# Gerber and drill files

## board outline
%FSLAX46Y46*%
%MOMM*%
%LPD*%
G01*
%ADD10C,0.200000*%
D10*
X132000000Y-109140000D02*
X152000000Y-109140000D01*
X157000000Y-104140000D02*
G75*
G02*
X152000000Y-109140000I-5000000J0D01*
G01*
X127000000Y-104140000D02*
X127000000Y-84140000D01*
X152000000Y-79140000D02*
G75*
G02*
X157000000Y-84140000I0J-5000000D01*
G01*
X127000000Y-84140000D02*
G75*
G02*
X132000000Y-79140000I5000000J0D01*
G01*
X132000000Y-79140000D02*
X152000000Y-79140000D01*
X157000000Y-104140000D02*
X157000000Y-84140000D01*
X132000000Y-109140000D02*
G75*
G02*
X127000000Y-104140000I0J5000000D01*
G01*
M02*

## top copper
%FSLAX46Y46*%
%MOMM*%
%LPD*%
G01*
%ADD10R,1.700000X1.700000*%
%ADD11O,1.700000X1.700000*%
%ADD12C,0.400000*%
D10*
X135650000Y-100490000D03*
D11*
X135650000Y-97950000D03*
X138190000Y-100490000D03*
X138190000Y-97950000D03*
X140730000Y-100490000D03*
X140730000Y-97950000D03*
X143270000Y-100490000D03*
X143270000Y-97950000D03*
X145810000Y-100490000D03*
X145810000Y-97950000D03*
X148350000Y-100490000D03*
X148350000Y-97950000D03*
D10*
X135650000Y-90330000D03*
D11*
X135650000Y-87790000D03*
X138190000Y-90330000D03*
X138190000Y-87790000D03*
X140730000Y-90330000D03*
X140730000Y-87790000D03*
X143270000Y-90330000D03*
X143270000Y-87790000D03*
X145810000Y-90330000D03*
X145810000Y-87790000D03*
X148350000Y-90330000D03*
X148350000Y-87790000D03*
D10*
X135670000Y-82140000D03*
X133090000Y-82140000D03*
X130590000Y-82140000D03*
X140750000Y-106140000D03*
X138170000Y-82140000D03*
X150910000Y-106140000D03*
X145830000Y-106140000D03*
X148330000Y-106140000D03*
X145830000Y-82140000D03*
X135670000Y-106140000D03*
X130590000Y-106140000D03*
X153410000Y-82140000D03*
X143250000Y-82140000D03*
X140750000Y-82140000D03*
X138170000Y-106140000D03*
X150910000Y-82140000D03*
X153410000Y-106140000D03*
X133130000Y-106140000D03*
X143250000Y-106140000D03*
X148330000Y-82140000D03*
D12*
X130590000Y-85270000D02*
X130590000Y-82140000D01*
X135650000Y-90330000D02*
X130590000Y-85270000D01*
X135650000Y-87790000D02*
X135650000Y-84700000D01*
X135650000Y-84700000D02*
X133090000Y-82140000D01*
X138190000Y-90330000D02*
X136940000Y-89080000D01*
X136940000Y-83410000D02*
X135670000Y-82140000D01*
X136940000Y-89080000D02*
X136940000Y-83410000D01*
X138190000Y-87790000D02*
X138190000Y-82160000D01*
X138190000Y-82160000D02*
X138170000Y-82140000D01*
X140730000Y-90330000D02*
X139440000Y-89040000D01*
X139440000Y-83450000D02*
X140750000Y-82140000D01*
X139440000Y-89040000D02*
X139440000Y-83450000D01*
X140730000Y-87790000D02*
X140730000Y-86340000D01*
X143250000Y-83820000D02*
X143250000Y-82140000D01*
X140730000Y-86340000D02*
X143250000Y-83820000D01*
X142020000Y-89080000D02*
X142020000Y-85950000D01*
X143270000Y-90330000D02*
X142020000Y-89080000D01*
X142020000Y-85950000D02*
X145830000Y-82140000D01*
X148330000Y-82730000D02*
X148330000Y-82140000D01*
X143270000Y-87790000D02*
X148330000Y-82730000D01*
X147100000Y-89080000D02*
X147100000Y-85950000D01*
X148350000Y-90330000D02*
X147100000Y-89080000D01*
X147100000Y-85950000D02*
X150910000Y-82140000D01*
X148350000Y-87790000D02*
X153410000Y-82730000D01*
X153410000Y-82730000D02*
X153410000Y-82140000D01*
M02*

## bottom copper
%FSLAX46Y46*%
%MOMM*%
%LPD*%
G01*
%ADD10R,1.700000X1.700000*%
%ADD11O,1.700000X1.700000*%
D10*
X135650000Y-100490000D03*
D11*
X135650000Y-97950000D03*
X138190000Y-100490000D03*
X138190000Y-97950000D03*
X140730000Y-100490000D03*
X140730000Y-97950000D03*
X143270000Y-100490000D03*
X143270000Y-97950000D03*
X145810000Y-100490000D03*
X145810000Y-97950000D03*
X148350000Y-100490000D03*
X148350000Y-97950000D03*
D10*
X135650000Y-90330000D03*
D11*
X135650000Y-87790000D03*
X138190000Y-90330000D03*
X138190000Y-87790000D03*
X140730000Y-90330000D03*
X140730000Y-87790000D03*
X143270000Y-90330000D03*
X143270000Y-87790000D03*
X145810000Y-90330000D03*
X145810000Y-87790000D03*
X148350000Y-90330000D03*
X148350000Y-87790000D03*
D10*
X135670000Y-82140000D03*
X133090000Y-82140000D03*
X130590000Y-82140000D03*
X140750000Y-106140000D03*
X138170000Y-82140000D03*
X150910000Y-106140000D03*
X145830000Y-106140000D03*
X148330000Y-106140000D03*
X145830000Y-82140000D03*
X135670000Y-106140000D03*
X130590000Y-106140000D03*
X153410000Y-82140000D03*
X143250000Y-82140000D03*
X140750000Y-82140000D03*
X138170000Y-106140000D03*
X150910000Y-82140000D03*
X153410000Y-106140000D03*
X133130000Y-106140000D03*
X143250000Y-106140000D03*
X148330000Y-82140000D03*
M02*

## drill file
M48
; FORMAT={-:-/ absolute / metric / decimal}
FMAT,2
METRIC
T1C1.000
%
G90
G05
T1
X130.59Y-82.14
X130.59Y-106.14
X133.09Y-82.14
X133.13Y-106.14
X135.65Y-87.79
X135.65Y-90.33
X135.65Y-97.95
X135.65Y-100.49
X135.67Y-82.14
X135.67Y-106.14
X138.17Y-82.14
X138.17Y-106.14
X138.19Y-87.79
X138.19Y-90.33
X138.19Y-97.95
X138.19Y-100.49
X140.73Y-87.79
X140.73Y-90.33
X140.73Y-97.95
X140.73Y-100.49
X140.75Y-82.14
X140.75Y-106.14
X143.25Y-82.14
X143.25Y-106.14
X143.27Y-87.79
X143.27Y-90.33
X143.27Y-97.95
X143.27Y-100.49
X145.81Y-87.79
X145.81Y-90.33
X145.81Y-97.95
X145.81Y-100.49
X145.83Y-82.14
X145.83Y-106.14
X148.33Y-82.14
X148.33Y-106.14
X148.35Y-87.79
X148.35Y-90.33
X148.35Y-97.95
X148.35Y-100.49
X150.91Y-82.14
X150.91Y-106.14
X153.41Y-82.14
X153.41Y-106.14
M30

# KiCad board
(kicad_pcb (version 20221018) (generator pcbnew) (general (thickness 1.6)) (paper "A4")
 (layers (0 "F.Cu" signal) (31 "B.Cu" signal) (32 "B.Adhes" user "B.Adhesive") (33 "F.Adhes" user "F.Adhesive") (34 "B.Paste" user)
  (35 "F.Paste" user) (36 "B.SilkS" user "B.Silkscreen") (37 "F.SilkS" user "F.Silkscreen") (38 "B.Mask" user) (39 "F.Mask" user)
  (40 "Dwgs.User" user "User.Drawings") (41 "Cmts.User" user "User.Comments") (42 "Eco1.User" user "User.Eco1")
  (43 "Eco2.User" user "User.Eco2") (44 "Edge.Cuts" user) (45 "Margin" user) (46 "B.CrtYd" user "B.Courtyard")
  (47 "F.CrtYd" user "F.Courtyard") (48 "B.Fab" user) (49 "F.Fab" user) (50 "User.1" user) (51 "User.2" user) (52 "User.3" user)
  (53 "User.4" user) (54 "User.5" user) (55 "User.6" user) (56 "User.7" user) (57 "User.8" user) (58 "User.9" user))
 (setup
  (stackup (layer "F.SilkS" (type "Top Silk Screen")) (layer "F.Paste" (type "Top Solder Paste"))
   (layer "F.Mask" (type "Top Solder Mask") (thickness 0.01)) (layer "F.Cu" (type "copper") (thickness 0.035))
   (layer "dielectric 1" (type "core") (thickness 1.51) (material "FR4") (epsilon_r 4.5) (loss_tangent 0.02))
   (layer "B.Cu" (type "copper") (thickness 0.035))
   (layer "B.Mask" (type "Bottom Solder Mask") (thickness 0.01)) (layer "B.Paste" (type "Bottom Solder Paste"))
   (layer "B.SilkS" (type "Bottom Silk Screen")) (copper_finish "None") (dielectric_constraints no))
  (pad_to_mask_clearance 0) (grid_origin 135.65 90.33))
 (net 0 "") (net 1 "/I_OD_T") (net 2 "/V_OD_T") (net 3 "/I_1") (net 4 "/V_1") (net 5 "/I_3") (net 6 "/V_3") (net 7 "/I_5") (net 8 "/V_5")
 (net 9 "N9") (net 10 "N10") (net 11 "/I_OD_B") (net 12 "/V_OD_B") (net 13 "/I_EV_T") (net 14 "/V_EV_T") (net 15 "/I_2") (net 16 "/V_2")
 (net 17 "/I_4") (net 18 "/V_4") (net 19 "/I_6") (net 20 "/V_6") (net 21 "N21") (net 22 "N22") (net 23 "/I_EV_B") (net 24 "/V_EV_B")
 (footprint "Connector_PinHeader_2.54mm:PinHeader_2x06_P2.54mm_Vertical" (layer "F.Cu") (at 135.65 100.49 90)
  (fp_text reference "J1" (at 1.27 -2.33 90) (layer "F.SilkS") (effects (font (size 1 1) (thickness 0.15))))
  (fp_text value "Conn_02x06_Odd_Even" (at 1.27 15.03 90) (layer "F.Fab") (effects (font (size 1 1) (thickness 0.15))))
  (pad "1" thru_hole rect (at 0 0 90) (size 1.7 1.7) (drill 1) (layers "*.Cu" "*.Mask") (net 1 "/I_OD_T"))
  (pad "2" thru_hole oval (at 2.54 0 90) (size 1.7 1.7) (drill 1) (layers "*.Cu" "*.Mask") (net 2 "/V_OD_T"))
  (pad "3" thru_hole oval (at 0 2.54 90) (size 1.7 1.7) (drill 1) (layers "*.Cu" "*.Mask") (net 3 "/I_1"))
  (pad "4" thru_hole oval (at 2.54 2.54 90) (size 1.7 1.7) (drill 1) (layers "*.Cu" "*.Mask") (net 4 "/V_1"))
  (pad "5" thru_hole oval (at 0 5.08 90) (size 1.7 1.7) (drill 1) (layers "*.Cu" "*.Mask") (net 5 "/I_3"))
  (pad "6" thru_hole oval (at 2.54 5.08 90) (size 1.7 1.7) (drill 1) (layers "*.Cu" "*.Mask") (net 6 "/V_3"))
  (pad "7" thru_hole oval (at 0 7.62 90) (size 1.7 1.7) (drill 1) (layers "*.Cu" "*.Mask") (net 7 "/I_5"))
  (pad "8" thru_hole oval (at 2.54 7.62 90) (size 1.7 1.7) (drill 1) (layers "*.Cu" "*.Mask") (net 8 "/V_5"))
  (pad "9" thru_hole oval (at 0 10.16 90) (size 1.7 1.7) (drill 1) (layers "*.Cu" "*.Mask") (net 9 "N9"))
  (pad "10" thru_hole oval (at 2.54 10.16 90) (size 1.7 1.7) (drill 1) (layers "*.Cu" "*.Mask") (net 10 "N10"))
  (pad "11" thru_hole oval (at 0 12.7 90) (size 1.7 1.7) (drill 1) (layers "*.Cu" "*.Mask") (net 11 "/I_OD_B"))
  (pad "12" thru_hole oval (at 2.54 12.7 90) (size 1.7 1.7) (drill 1) (layers "*.Cu" "*.Mask") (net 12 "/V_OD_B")))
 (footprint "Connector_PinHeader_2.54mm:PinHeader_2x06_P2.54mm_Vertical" (layer "F.Cu") (at 135.65 90.33 90)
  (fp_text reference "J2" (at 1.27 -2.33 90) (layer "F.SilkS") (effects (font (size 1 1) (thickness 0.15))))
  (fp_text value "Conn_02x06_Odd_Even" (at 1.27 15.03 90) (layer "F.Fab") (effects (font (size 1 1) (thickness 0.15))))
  (pad "1" thru_hole rect (at 0 0 90) (size 1.7 1.7) (drill 1) (layers "*.Cu" "*.Mask") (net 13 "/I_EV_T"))
  (pad "2" thru_hole oval (at 2.54 0 90) (size 1.7 1.7) (drill 1) (layers "*.Cu" "*.Mask") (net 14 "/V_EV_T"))
  (pad "3" thru_hole oval (at 0 2.54 90) (size 1.7 1.7) (drill 1) (layers "*.Cu" "*.Mask") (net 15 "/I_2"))
  (pad "4" thru_hole oval (at 2.54 2.54 90) (size 1.7 1.7) (drill 1) (layers "*.Cu" "*.Mask") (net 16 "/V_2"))
  (pad "5" thru_hole oval (at 0 5.08 90) (size 1.7 1.7) (drill 1) (layers "*.Cu" "*.Mask") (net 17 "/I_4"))
  (pad "6" thru_hole oval (at 2.54 5.08 90) (size 1.7 1.7) (drill 1) (layers "*.Cu" "*.Mask") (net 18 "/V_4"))
  (pad "7" thru_hole oval (at 0 7.62 90) (size 1.7 1.7) (drill 1) (layers "*.Cu" "*.Mask") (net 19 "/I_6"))
  (pad "8" thru_hole oval (at 2.54 7.62 90) (size 1.7 1.7) (drill 1) (layers "*.Cu" "*.Mask") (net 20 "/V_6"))
  (pad "9" thru_hole oval (at 0 10.16 90) (size 1.7 1.7) (drill 1) (layers "*.Cu" "*.Mask") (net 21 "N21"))
  (pad "10" thru_hole oval (at 2.54 10.16 90) (size 1.7 1.7) (drill 1) (layers "*.Cu" "*.Mask") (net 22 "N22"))
  (pad "11" thru_hole oval (at 0 12.7 90) (size 1.7 1.7) (drill 1) (layers "*.Cu" "*.Mask") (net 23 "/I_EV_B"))
  (pad "12" thru_hole oval (at 2.54 12.7 90) (size 1.7 1.7) (drill 1) (layers "*.Cu" "*.Mask") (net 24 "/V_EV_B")))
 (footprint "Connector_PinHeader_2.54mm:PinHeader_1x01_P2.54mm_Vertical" (layer "B.Cu") (at 135.67 82.14 180)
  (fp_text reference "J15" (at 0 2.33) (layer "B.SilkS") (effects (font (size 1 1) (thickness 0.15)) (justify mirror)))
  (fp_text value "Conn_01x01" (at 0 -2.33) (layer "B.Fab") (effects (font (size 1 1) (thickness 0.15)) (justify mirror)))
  (pad "1" thru_hole rect (at 0 0 180) (size 1.7 1.7) (drill 1) (layers "*.Cu" "*.Mask") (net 15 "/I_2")))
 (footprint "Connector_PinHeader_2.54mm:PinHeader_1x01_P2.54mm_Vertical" (layer "B.Cu") (at 133.09 82.14 180)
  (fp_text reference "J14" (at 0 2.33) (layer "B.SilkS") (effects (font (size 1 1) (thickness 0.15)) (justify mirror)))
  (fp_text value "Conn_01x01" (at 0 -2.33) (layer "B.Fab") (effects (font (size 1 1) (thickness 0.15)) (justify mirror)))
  (pad "1" thru_hole rect (at 0 0 180) (size 1.7 1.7) (drill 1) (layers "*.Cu" "*.Mask") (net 14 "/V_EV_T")))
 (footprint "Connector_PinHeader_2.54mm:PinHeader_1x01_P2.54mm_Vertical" (layer "B.Cu") (at 130.59 82.14 180)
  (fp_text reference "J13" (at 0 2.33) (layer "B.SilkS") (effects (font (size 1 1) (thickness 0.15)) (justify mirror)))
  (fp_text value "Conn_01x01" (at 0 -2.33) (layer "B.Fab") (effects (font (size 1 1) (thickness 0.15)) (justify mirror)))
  (pad "1" thru_hole rect (at 0 0 180) (size 1.7 1.7) (drill 1) (layers "*.Cu" "*.Mask") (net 13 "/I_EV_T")))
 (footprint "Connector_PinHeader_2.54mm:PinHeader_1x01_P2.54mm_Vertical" (layer "B.Cu") (at 140.75 106.14 180)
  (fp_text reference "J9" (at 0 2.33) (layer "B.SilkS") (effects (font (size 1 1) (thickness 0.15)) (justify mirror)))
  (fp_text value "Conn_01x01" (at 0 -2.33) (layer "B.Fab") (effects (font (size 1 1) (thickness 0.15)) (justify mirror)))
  (pad "1" thru_hole rect (at 0 0 180) (size 1.7 1.7) (drill 1) (layers "*.Cu" "*.Mask") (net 5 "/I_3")))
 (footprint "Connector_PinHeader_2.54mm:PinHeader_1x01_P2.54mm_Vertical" (layer "B.Cu") (at 138.17 82.14 180)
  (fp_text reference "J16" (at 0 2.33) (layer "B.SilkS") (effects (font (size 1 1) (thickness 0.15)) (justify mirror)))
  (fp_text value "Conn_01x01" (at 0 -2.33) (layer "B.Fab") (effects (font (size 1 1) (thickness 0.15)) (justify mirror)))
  (pad "1" thru_hole rect (at 0 0 180) (size 1.7 1.7) (drill 1) (layers "*.Cu" "*.Mask") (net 16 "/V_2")))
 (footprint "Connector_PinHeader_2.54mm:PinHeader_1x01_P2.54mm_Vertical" (layer "B.Cu") (at 150.91 106.14 180)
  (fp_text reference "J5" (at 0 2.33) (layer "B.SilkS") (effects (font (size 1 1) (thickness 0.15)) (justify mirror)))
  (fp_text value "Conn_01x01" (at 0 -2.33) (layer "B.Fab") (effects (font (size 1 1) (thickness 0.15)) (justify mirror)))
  (pad "1" thru_hole rect (at 0 0 180) (size 1.7 1.7) (drill 1) (layers "*.Cu" "*.Mask") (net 11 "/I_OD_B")))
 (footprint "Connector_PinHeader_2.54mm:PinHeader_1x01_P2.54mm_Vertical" (layer "B.Cu") (at 145.83 106.14 180)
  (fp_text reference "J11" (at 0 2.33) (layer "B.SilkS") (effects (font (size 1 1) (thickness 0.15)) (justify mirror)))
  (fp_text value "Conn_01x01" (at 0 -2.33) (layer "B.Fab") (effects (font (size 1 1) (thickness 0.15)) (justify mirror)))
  (pad "1" thru_hole rect (at 0 0 180) (size 1.7 1.7) (drill 1) (layers "*.Cu" "*.Mask") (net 7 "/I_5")))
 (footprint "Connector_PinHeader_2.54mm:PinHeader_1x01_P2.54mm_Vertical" (layer "B.Cu") (at 148.33 106.14 180)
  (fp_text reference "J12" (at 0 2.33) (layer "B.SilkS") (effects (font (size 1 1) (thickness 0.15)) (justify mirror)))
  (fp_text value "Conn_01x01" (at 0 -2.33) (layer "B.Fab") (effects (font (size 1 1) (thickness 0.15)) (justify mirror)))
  (pad "1" thru_hole rect (at 0 0 180) (size 1.7 1.7) (drill 1) (layers "*.Cu" "*.Mask") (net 8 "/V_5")))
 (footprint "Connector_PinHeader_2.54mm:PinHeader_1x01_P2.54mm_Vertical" (layer "B.Cu") (at 145.83 82.14 180)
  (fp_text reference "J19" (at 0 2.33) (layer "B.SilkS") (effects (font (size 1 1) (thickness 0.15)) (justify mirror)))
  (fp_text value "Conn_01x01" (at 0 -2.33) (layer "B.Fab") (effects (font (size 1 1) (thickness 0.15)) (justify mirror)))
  (pad "1" thru_hole rect (at 0 0 180) (size 1.7 1.7) (drill 1) (layers "*.Cu" "*.Mask") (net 19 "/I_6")))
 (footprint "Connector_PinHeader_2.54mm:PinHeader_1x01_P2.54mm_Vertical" (layer "B.Cu") (at 135.67 106.14 180)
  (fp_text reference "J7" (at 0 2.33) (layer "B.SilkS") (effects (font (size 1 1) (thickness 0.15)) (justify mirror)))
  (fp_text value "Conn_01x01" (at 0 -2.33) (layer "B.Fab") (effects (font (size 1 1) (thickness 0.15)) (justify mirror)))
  (pad "1" thru_hole rect (at 0 0 180) (size 1.7 1.7) (drill 1) (layers "*.Cu" "*.Mask") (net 3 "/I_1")))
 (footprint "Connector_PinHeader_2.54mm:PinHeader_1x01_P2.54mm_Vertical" (layer "B.Cu") (at 130.59 106.14 180)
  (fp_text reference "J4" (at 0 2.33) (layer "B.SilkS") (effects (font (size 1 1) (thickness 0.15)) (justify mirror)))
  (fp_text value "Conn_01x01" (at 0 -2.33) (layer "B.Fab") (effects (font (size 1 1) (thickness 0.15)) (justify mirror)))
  (pad "1" thru_hole rect (at 0 0 180) (size 1.7 1.7) (drill 1) (layers "*.Cu" "*.Mask") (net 1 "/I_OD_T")))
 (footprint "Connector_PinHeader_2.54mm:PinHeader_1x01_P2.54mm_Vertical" (layer "B.Cu") (at 153.41 82.14 180)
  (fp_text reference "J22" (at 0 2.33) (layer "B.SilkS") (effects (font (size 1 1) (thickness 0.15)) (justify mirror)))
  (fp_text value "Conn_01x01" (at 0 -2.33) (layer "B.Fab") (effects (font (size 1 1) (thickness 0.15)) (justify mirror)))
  (pad "1" thru_hole rect (at 0 0 180) (size 1.7 1.7) (drill 1) (layers "*.Cu" "*.Mask") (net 24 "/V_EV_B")))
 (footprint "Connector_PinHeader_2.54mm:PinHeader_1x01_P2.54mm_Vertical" (layer "B.Cu") (at 143.25 82.14 180)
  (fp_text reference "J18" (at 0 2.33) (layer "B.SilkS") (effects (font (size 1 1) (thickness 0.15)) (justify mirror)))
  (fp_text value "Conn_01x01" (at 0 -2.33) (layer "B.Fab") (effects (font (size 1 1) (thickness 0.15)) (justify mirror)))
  (pad "1" thru_hole rect (at 0 0 180) (size 1.7 1.7) (drill 1) (layers "*.Cu" "*.Mask") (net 18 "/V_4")))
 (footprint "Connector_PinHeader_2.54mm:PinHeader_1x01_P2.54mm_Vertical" (layer "B.Cu") (at 140.75 82.14 180)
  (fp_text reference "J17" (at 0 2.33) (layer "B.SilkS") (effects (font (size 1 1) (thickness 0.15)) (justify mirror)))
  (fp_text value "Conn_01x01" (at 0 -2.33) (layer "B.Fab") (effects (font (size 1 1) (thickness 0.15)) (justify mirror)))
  (pad "1" thru_hole rect (at 0 0 180) (size 1.7 1.7) (drill 1) (layers "*.Cu" "*.Mask") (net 17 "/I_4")))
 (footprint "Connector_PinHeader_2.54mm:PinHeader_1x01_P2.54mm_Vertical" (layer "B.Cu") (at 138.17 106.14 180)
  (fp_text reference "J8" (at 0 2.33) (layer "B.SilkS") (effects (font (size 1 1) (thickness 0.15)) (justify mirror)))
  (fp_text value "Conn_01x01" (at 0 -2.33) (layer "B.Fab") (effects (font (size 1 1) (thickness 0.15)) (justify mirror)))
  (pad "1" thru_hole rect (at 0 0 180) (size 1.7 1.7) (drill 1) (layers "*.Cu" "*.Mask") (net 4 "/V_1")))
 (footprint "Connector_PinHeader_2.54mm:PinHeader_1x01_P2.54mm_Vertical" (layer "B.Cu") (at 150.91 82.14 180)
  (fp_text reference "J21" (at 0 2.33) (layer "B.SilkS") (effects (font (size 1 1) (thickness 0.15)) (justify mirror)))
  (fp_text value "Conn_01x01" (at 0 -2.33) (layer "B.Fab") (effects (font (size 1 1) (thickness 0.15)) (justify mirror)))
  (pad "1" thru_hole rect (at 0 0 180) (size 1.7 1.7) (drill 1) (layers "*.Cu" "*.Mask") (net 23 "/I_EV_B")))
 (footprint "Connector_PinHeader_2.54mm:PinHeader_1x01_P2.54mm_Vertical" (layer "B.Cu") (at 153.41 106.14 180)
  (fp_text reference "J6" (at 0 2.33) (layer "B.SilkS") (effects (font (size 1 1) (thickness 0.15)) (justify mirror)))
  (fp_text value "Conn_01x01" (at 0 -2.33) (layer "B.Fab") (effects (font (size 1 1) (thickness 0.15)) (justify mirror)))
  (pad "1" thru_hole rect (at 0 0 180) (size 1.7 1.7) (drill 1) (layers "*.Cu" "*.Mask") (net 12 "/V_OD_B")))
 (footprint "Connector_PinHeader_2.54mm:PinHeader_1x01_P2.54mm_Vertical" (layer "B.Cu") (at 133.13 106.14 180)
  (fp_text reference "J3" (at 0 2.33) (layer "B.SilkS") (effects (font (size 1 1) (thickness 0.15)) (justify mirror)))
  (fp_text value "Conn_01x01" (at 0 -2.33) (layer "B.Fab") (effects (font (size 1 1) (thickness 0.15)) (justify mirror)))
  (pad "1" thru_hole rect (at 0 0 180) (size 1.7 1.7) (drill 1) (layers "*.Cu" "*.Mask") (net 2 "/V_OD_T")))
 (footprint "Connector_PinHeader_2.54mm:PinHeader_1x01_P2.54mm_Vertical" (layer "B.Cu") (at 143.25 106.14 180)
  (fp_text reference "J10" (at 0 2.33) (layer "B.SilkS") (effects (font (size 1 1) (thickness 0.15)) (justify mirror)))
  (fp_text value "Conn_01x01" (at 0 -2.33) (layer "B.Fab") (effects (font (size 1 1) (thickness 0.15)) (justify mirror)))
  (pad "1" thru_hole rect (at 0 0 180) (size 1.7 1.7) (drill 1) (layers "*.Cu" "*.Mask") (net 6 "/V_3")))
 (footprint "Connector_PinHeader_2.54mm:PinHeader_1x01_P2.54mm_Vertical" (layer "B.Cu") (at 148.33 82.14 180)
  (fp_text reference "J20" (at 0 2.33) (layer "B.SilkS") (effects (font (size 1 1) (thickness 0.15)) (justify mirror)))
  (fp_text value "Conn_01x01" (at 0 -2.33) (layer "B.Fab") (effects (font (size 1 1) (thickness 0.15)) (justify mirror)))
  (pad "1" thru_hole rect (at 0 0 180) (size 1.7 1.7) (drill 1) (layers "*.Cu" "*.Mask") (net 20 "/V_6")))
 (gr_line (start 132 109.14) (end 152 109.14) (stroke (width 0.2) (type solid)) (layer "Edge.Cuts"))
 (gr_arc (start 157 104.14) (mid 155.535534 107.675533) (end 152 109.14) (stroke (width 0.2) (type solid)) (layer "Edge.Cuts"))
 (gr_line (start 127 104.14) (end 127 84.14) (stroke (width 0.2) (type solid)) (layer "Edge.Cuts"))
 (gr_arc (start 152 79.14) (mid 155.535533 80.604466) (end 157 84.14) (stroke (width 0.2) (type solid)) (layer "Edge.Cuts"))
 (gr_arc (start 127 84.14) (mid 128.464466 80.604467) (end 132 79.14) (stroke (width 0.2) (type solid)) (layer "Edge.Cuts"))
 (gr_line (start 132 79.14) (end 152 79.14) (stroke (width 0.2) (type solid)) (layer "Edge.Cuts"))
 (gr_line (start 157 104.14) (end 157 84.14) (stroke (width 0.2) (type solid)) (layer "Edge.Cuts"))
 (gr_arc (start 132 109.14) (mid 128.464467 107.675534) (end 127 104.14) (stroke (width 0.2) (type solid)) (layer "Edge.Cuts"))
 (segment (start 130.59 85.27) (end 130.59 82.14) (width 0.4) (layer "F.Cu") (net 13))
 (segment (start 135.65 90.33) (end 130.59 85.27) (width 0.4) (layer "F.Cu") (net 13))
 (segment (start 135.65 87.79) (end 135.65 84.7) (width 0.4) (layer "F.Cu") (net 14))
 (segment (start 135.65 84.7) (end 133.09 82.14) (width 0.4) (layer "F.Cu") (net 14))
 (segment (start 138.19 90.33) (end 136.94 89.08) (width 0.4) (layer "F.Cu") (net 15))
 (segment (start 136.94 83.41) (end 135.67 82.14) (width 0.4) (layer "F.Cu") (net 15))
 (segment (start 136.94 89.08) (end 136.94 83.41) (width 0.4) (layer "F.Cu") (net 15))
 (segment (start 138.19 87.79) (end 138.19 82.16) (width 0.4) (layer "F.Cu") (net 16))
 (segment (start 138.19 82.16) (end 138.17 82.14) (width 0.4) (layer "F.Cu") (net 16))
 (segment (start 140.73 90.33) (end 139.44 89.04) (width 0.4) (layer "F.Cu") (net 17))
 (segment (start 139.44 83.45) (end 140.75 82.14) (width 0.4) (layer "F.Cu") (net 17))
 (segment (start 139.44 89.04) (end 139.44 83.45) (width 0.4) (layer "F.Cu") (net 17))
 (segment (start 140.73 87.79) (end 140.73 86.34) (width 0.4) (layer "F.Cu") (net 18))
 (segment (start 143.25 83.82) (end 143.25 82.14) (width 0.4) (layer "F.Cu") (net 18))
 (segment (start 140.73 86.34) (end 143.25 83.82) (width 0.4) (layer "F.Cu") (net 18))
 (segment (start 142.02 89.08) (end 142.02 85.95) (width 0.4) (layer "F.Cu") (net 19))
 (segment (start 143.27 90.33) (end 142.02 89.08) (width 0.4) (layer "F.Cu") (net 19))
 (segment (start 142.02 85.95) (end 145.83 82.14) (width 0.4) (layer "F.Cu") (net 19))
 (segment (start 148.33 82.73) (end 148.33 82.14) (width 0.4) (layer "F.Cu") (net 20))
 (segment (start 143.27 87.79) (end 148.33 82.73) (width 0.4) (layer "F.Cu") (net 20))
 (segment (start 147.1 89.08) (end 147.1 85.95) (width 0.4) (layer "F.Cu") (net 23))
 (segment (start 148.35 90.33) (end 147.1 89.08) (width 0.4) (layer "F.Cu") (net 23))
 (segment (start 147.1 85.95) (end 150.91 82.14) (width 0.4) (layer "F.Cu") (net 23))
 (segment (start 148.35 87.79) (end 153.41 82.73) (width 0.4) (layer "F.Cu") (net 24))
 (segment (start 153.41 82.73) (end 153.41 82.14) (width 0.4) (layer "F.Cu") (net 24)))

